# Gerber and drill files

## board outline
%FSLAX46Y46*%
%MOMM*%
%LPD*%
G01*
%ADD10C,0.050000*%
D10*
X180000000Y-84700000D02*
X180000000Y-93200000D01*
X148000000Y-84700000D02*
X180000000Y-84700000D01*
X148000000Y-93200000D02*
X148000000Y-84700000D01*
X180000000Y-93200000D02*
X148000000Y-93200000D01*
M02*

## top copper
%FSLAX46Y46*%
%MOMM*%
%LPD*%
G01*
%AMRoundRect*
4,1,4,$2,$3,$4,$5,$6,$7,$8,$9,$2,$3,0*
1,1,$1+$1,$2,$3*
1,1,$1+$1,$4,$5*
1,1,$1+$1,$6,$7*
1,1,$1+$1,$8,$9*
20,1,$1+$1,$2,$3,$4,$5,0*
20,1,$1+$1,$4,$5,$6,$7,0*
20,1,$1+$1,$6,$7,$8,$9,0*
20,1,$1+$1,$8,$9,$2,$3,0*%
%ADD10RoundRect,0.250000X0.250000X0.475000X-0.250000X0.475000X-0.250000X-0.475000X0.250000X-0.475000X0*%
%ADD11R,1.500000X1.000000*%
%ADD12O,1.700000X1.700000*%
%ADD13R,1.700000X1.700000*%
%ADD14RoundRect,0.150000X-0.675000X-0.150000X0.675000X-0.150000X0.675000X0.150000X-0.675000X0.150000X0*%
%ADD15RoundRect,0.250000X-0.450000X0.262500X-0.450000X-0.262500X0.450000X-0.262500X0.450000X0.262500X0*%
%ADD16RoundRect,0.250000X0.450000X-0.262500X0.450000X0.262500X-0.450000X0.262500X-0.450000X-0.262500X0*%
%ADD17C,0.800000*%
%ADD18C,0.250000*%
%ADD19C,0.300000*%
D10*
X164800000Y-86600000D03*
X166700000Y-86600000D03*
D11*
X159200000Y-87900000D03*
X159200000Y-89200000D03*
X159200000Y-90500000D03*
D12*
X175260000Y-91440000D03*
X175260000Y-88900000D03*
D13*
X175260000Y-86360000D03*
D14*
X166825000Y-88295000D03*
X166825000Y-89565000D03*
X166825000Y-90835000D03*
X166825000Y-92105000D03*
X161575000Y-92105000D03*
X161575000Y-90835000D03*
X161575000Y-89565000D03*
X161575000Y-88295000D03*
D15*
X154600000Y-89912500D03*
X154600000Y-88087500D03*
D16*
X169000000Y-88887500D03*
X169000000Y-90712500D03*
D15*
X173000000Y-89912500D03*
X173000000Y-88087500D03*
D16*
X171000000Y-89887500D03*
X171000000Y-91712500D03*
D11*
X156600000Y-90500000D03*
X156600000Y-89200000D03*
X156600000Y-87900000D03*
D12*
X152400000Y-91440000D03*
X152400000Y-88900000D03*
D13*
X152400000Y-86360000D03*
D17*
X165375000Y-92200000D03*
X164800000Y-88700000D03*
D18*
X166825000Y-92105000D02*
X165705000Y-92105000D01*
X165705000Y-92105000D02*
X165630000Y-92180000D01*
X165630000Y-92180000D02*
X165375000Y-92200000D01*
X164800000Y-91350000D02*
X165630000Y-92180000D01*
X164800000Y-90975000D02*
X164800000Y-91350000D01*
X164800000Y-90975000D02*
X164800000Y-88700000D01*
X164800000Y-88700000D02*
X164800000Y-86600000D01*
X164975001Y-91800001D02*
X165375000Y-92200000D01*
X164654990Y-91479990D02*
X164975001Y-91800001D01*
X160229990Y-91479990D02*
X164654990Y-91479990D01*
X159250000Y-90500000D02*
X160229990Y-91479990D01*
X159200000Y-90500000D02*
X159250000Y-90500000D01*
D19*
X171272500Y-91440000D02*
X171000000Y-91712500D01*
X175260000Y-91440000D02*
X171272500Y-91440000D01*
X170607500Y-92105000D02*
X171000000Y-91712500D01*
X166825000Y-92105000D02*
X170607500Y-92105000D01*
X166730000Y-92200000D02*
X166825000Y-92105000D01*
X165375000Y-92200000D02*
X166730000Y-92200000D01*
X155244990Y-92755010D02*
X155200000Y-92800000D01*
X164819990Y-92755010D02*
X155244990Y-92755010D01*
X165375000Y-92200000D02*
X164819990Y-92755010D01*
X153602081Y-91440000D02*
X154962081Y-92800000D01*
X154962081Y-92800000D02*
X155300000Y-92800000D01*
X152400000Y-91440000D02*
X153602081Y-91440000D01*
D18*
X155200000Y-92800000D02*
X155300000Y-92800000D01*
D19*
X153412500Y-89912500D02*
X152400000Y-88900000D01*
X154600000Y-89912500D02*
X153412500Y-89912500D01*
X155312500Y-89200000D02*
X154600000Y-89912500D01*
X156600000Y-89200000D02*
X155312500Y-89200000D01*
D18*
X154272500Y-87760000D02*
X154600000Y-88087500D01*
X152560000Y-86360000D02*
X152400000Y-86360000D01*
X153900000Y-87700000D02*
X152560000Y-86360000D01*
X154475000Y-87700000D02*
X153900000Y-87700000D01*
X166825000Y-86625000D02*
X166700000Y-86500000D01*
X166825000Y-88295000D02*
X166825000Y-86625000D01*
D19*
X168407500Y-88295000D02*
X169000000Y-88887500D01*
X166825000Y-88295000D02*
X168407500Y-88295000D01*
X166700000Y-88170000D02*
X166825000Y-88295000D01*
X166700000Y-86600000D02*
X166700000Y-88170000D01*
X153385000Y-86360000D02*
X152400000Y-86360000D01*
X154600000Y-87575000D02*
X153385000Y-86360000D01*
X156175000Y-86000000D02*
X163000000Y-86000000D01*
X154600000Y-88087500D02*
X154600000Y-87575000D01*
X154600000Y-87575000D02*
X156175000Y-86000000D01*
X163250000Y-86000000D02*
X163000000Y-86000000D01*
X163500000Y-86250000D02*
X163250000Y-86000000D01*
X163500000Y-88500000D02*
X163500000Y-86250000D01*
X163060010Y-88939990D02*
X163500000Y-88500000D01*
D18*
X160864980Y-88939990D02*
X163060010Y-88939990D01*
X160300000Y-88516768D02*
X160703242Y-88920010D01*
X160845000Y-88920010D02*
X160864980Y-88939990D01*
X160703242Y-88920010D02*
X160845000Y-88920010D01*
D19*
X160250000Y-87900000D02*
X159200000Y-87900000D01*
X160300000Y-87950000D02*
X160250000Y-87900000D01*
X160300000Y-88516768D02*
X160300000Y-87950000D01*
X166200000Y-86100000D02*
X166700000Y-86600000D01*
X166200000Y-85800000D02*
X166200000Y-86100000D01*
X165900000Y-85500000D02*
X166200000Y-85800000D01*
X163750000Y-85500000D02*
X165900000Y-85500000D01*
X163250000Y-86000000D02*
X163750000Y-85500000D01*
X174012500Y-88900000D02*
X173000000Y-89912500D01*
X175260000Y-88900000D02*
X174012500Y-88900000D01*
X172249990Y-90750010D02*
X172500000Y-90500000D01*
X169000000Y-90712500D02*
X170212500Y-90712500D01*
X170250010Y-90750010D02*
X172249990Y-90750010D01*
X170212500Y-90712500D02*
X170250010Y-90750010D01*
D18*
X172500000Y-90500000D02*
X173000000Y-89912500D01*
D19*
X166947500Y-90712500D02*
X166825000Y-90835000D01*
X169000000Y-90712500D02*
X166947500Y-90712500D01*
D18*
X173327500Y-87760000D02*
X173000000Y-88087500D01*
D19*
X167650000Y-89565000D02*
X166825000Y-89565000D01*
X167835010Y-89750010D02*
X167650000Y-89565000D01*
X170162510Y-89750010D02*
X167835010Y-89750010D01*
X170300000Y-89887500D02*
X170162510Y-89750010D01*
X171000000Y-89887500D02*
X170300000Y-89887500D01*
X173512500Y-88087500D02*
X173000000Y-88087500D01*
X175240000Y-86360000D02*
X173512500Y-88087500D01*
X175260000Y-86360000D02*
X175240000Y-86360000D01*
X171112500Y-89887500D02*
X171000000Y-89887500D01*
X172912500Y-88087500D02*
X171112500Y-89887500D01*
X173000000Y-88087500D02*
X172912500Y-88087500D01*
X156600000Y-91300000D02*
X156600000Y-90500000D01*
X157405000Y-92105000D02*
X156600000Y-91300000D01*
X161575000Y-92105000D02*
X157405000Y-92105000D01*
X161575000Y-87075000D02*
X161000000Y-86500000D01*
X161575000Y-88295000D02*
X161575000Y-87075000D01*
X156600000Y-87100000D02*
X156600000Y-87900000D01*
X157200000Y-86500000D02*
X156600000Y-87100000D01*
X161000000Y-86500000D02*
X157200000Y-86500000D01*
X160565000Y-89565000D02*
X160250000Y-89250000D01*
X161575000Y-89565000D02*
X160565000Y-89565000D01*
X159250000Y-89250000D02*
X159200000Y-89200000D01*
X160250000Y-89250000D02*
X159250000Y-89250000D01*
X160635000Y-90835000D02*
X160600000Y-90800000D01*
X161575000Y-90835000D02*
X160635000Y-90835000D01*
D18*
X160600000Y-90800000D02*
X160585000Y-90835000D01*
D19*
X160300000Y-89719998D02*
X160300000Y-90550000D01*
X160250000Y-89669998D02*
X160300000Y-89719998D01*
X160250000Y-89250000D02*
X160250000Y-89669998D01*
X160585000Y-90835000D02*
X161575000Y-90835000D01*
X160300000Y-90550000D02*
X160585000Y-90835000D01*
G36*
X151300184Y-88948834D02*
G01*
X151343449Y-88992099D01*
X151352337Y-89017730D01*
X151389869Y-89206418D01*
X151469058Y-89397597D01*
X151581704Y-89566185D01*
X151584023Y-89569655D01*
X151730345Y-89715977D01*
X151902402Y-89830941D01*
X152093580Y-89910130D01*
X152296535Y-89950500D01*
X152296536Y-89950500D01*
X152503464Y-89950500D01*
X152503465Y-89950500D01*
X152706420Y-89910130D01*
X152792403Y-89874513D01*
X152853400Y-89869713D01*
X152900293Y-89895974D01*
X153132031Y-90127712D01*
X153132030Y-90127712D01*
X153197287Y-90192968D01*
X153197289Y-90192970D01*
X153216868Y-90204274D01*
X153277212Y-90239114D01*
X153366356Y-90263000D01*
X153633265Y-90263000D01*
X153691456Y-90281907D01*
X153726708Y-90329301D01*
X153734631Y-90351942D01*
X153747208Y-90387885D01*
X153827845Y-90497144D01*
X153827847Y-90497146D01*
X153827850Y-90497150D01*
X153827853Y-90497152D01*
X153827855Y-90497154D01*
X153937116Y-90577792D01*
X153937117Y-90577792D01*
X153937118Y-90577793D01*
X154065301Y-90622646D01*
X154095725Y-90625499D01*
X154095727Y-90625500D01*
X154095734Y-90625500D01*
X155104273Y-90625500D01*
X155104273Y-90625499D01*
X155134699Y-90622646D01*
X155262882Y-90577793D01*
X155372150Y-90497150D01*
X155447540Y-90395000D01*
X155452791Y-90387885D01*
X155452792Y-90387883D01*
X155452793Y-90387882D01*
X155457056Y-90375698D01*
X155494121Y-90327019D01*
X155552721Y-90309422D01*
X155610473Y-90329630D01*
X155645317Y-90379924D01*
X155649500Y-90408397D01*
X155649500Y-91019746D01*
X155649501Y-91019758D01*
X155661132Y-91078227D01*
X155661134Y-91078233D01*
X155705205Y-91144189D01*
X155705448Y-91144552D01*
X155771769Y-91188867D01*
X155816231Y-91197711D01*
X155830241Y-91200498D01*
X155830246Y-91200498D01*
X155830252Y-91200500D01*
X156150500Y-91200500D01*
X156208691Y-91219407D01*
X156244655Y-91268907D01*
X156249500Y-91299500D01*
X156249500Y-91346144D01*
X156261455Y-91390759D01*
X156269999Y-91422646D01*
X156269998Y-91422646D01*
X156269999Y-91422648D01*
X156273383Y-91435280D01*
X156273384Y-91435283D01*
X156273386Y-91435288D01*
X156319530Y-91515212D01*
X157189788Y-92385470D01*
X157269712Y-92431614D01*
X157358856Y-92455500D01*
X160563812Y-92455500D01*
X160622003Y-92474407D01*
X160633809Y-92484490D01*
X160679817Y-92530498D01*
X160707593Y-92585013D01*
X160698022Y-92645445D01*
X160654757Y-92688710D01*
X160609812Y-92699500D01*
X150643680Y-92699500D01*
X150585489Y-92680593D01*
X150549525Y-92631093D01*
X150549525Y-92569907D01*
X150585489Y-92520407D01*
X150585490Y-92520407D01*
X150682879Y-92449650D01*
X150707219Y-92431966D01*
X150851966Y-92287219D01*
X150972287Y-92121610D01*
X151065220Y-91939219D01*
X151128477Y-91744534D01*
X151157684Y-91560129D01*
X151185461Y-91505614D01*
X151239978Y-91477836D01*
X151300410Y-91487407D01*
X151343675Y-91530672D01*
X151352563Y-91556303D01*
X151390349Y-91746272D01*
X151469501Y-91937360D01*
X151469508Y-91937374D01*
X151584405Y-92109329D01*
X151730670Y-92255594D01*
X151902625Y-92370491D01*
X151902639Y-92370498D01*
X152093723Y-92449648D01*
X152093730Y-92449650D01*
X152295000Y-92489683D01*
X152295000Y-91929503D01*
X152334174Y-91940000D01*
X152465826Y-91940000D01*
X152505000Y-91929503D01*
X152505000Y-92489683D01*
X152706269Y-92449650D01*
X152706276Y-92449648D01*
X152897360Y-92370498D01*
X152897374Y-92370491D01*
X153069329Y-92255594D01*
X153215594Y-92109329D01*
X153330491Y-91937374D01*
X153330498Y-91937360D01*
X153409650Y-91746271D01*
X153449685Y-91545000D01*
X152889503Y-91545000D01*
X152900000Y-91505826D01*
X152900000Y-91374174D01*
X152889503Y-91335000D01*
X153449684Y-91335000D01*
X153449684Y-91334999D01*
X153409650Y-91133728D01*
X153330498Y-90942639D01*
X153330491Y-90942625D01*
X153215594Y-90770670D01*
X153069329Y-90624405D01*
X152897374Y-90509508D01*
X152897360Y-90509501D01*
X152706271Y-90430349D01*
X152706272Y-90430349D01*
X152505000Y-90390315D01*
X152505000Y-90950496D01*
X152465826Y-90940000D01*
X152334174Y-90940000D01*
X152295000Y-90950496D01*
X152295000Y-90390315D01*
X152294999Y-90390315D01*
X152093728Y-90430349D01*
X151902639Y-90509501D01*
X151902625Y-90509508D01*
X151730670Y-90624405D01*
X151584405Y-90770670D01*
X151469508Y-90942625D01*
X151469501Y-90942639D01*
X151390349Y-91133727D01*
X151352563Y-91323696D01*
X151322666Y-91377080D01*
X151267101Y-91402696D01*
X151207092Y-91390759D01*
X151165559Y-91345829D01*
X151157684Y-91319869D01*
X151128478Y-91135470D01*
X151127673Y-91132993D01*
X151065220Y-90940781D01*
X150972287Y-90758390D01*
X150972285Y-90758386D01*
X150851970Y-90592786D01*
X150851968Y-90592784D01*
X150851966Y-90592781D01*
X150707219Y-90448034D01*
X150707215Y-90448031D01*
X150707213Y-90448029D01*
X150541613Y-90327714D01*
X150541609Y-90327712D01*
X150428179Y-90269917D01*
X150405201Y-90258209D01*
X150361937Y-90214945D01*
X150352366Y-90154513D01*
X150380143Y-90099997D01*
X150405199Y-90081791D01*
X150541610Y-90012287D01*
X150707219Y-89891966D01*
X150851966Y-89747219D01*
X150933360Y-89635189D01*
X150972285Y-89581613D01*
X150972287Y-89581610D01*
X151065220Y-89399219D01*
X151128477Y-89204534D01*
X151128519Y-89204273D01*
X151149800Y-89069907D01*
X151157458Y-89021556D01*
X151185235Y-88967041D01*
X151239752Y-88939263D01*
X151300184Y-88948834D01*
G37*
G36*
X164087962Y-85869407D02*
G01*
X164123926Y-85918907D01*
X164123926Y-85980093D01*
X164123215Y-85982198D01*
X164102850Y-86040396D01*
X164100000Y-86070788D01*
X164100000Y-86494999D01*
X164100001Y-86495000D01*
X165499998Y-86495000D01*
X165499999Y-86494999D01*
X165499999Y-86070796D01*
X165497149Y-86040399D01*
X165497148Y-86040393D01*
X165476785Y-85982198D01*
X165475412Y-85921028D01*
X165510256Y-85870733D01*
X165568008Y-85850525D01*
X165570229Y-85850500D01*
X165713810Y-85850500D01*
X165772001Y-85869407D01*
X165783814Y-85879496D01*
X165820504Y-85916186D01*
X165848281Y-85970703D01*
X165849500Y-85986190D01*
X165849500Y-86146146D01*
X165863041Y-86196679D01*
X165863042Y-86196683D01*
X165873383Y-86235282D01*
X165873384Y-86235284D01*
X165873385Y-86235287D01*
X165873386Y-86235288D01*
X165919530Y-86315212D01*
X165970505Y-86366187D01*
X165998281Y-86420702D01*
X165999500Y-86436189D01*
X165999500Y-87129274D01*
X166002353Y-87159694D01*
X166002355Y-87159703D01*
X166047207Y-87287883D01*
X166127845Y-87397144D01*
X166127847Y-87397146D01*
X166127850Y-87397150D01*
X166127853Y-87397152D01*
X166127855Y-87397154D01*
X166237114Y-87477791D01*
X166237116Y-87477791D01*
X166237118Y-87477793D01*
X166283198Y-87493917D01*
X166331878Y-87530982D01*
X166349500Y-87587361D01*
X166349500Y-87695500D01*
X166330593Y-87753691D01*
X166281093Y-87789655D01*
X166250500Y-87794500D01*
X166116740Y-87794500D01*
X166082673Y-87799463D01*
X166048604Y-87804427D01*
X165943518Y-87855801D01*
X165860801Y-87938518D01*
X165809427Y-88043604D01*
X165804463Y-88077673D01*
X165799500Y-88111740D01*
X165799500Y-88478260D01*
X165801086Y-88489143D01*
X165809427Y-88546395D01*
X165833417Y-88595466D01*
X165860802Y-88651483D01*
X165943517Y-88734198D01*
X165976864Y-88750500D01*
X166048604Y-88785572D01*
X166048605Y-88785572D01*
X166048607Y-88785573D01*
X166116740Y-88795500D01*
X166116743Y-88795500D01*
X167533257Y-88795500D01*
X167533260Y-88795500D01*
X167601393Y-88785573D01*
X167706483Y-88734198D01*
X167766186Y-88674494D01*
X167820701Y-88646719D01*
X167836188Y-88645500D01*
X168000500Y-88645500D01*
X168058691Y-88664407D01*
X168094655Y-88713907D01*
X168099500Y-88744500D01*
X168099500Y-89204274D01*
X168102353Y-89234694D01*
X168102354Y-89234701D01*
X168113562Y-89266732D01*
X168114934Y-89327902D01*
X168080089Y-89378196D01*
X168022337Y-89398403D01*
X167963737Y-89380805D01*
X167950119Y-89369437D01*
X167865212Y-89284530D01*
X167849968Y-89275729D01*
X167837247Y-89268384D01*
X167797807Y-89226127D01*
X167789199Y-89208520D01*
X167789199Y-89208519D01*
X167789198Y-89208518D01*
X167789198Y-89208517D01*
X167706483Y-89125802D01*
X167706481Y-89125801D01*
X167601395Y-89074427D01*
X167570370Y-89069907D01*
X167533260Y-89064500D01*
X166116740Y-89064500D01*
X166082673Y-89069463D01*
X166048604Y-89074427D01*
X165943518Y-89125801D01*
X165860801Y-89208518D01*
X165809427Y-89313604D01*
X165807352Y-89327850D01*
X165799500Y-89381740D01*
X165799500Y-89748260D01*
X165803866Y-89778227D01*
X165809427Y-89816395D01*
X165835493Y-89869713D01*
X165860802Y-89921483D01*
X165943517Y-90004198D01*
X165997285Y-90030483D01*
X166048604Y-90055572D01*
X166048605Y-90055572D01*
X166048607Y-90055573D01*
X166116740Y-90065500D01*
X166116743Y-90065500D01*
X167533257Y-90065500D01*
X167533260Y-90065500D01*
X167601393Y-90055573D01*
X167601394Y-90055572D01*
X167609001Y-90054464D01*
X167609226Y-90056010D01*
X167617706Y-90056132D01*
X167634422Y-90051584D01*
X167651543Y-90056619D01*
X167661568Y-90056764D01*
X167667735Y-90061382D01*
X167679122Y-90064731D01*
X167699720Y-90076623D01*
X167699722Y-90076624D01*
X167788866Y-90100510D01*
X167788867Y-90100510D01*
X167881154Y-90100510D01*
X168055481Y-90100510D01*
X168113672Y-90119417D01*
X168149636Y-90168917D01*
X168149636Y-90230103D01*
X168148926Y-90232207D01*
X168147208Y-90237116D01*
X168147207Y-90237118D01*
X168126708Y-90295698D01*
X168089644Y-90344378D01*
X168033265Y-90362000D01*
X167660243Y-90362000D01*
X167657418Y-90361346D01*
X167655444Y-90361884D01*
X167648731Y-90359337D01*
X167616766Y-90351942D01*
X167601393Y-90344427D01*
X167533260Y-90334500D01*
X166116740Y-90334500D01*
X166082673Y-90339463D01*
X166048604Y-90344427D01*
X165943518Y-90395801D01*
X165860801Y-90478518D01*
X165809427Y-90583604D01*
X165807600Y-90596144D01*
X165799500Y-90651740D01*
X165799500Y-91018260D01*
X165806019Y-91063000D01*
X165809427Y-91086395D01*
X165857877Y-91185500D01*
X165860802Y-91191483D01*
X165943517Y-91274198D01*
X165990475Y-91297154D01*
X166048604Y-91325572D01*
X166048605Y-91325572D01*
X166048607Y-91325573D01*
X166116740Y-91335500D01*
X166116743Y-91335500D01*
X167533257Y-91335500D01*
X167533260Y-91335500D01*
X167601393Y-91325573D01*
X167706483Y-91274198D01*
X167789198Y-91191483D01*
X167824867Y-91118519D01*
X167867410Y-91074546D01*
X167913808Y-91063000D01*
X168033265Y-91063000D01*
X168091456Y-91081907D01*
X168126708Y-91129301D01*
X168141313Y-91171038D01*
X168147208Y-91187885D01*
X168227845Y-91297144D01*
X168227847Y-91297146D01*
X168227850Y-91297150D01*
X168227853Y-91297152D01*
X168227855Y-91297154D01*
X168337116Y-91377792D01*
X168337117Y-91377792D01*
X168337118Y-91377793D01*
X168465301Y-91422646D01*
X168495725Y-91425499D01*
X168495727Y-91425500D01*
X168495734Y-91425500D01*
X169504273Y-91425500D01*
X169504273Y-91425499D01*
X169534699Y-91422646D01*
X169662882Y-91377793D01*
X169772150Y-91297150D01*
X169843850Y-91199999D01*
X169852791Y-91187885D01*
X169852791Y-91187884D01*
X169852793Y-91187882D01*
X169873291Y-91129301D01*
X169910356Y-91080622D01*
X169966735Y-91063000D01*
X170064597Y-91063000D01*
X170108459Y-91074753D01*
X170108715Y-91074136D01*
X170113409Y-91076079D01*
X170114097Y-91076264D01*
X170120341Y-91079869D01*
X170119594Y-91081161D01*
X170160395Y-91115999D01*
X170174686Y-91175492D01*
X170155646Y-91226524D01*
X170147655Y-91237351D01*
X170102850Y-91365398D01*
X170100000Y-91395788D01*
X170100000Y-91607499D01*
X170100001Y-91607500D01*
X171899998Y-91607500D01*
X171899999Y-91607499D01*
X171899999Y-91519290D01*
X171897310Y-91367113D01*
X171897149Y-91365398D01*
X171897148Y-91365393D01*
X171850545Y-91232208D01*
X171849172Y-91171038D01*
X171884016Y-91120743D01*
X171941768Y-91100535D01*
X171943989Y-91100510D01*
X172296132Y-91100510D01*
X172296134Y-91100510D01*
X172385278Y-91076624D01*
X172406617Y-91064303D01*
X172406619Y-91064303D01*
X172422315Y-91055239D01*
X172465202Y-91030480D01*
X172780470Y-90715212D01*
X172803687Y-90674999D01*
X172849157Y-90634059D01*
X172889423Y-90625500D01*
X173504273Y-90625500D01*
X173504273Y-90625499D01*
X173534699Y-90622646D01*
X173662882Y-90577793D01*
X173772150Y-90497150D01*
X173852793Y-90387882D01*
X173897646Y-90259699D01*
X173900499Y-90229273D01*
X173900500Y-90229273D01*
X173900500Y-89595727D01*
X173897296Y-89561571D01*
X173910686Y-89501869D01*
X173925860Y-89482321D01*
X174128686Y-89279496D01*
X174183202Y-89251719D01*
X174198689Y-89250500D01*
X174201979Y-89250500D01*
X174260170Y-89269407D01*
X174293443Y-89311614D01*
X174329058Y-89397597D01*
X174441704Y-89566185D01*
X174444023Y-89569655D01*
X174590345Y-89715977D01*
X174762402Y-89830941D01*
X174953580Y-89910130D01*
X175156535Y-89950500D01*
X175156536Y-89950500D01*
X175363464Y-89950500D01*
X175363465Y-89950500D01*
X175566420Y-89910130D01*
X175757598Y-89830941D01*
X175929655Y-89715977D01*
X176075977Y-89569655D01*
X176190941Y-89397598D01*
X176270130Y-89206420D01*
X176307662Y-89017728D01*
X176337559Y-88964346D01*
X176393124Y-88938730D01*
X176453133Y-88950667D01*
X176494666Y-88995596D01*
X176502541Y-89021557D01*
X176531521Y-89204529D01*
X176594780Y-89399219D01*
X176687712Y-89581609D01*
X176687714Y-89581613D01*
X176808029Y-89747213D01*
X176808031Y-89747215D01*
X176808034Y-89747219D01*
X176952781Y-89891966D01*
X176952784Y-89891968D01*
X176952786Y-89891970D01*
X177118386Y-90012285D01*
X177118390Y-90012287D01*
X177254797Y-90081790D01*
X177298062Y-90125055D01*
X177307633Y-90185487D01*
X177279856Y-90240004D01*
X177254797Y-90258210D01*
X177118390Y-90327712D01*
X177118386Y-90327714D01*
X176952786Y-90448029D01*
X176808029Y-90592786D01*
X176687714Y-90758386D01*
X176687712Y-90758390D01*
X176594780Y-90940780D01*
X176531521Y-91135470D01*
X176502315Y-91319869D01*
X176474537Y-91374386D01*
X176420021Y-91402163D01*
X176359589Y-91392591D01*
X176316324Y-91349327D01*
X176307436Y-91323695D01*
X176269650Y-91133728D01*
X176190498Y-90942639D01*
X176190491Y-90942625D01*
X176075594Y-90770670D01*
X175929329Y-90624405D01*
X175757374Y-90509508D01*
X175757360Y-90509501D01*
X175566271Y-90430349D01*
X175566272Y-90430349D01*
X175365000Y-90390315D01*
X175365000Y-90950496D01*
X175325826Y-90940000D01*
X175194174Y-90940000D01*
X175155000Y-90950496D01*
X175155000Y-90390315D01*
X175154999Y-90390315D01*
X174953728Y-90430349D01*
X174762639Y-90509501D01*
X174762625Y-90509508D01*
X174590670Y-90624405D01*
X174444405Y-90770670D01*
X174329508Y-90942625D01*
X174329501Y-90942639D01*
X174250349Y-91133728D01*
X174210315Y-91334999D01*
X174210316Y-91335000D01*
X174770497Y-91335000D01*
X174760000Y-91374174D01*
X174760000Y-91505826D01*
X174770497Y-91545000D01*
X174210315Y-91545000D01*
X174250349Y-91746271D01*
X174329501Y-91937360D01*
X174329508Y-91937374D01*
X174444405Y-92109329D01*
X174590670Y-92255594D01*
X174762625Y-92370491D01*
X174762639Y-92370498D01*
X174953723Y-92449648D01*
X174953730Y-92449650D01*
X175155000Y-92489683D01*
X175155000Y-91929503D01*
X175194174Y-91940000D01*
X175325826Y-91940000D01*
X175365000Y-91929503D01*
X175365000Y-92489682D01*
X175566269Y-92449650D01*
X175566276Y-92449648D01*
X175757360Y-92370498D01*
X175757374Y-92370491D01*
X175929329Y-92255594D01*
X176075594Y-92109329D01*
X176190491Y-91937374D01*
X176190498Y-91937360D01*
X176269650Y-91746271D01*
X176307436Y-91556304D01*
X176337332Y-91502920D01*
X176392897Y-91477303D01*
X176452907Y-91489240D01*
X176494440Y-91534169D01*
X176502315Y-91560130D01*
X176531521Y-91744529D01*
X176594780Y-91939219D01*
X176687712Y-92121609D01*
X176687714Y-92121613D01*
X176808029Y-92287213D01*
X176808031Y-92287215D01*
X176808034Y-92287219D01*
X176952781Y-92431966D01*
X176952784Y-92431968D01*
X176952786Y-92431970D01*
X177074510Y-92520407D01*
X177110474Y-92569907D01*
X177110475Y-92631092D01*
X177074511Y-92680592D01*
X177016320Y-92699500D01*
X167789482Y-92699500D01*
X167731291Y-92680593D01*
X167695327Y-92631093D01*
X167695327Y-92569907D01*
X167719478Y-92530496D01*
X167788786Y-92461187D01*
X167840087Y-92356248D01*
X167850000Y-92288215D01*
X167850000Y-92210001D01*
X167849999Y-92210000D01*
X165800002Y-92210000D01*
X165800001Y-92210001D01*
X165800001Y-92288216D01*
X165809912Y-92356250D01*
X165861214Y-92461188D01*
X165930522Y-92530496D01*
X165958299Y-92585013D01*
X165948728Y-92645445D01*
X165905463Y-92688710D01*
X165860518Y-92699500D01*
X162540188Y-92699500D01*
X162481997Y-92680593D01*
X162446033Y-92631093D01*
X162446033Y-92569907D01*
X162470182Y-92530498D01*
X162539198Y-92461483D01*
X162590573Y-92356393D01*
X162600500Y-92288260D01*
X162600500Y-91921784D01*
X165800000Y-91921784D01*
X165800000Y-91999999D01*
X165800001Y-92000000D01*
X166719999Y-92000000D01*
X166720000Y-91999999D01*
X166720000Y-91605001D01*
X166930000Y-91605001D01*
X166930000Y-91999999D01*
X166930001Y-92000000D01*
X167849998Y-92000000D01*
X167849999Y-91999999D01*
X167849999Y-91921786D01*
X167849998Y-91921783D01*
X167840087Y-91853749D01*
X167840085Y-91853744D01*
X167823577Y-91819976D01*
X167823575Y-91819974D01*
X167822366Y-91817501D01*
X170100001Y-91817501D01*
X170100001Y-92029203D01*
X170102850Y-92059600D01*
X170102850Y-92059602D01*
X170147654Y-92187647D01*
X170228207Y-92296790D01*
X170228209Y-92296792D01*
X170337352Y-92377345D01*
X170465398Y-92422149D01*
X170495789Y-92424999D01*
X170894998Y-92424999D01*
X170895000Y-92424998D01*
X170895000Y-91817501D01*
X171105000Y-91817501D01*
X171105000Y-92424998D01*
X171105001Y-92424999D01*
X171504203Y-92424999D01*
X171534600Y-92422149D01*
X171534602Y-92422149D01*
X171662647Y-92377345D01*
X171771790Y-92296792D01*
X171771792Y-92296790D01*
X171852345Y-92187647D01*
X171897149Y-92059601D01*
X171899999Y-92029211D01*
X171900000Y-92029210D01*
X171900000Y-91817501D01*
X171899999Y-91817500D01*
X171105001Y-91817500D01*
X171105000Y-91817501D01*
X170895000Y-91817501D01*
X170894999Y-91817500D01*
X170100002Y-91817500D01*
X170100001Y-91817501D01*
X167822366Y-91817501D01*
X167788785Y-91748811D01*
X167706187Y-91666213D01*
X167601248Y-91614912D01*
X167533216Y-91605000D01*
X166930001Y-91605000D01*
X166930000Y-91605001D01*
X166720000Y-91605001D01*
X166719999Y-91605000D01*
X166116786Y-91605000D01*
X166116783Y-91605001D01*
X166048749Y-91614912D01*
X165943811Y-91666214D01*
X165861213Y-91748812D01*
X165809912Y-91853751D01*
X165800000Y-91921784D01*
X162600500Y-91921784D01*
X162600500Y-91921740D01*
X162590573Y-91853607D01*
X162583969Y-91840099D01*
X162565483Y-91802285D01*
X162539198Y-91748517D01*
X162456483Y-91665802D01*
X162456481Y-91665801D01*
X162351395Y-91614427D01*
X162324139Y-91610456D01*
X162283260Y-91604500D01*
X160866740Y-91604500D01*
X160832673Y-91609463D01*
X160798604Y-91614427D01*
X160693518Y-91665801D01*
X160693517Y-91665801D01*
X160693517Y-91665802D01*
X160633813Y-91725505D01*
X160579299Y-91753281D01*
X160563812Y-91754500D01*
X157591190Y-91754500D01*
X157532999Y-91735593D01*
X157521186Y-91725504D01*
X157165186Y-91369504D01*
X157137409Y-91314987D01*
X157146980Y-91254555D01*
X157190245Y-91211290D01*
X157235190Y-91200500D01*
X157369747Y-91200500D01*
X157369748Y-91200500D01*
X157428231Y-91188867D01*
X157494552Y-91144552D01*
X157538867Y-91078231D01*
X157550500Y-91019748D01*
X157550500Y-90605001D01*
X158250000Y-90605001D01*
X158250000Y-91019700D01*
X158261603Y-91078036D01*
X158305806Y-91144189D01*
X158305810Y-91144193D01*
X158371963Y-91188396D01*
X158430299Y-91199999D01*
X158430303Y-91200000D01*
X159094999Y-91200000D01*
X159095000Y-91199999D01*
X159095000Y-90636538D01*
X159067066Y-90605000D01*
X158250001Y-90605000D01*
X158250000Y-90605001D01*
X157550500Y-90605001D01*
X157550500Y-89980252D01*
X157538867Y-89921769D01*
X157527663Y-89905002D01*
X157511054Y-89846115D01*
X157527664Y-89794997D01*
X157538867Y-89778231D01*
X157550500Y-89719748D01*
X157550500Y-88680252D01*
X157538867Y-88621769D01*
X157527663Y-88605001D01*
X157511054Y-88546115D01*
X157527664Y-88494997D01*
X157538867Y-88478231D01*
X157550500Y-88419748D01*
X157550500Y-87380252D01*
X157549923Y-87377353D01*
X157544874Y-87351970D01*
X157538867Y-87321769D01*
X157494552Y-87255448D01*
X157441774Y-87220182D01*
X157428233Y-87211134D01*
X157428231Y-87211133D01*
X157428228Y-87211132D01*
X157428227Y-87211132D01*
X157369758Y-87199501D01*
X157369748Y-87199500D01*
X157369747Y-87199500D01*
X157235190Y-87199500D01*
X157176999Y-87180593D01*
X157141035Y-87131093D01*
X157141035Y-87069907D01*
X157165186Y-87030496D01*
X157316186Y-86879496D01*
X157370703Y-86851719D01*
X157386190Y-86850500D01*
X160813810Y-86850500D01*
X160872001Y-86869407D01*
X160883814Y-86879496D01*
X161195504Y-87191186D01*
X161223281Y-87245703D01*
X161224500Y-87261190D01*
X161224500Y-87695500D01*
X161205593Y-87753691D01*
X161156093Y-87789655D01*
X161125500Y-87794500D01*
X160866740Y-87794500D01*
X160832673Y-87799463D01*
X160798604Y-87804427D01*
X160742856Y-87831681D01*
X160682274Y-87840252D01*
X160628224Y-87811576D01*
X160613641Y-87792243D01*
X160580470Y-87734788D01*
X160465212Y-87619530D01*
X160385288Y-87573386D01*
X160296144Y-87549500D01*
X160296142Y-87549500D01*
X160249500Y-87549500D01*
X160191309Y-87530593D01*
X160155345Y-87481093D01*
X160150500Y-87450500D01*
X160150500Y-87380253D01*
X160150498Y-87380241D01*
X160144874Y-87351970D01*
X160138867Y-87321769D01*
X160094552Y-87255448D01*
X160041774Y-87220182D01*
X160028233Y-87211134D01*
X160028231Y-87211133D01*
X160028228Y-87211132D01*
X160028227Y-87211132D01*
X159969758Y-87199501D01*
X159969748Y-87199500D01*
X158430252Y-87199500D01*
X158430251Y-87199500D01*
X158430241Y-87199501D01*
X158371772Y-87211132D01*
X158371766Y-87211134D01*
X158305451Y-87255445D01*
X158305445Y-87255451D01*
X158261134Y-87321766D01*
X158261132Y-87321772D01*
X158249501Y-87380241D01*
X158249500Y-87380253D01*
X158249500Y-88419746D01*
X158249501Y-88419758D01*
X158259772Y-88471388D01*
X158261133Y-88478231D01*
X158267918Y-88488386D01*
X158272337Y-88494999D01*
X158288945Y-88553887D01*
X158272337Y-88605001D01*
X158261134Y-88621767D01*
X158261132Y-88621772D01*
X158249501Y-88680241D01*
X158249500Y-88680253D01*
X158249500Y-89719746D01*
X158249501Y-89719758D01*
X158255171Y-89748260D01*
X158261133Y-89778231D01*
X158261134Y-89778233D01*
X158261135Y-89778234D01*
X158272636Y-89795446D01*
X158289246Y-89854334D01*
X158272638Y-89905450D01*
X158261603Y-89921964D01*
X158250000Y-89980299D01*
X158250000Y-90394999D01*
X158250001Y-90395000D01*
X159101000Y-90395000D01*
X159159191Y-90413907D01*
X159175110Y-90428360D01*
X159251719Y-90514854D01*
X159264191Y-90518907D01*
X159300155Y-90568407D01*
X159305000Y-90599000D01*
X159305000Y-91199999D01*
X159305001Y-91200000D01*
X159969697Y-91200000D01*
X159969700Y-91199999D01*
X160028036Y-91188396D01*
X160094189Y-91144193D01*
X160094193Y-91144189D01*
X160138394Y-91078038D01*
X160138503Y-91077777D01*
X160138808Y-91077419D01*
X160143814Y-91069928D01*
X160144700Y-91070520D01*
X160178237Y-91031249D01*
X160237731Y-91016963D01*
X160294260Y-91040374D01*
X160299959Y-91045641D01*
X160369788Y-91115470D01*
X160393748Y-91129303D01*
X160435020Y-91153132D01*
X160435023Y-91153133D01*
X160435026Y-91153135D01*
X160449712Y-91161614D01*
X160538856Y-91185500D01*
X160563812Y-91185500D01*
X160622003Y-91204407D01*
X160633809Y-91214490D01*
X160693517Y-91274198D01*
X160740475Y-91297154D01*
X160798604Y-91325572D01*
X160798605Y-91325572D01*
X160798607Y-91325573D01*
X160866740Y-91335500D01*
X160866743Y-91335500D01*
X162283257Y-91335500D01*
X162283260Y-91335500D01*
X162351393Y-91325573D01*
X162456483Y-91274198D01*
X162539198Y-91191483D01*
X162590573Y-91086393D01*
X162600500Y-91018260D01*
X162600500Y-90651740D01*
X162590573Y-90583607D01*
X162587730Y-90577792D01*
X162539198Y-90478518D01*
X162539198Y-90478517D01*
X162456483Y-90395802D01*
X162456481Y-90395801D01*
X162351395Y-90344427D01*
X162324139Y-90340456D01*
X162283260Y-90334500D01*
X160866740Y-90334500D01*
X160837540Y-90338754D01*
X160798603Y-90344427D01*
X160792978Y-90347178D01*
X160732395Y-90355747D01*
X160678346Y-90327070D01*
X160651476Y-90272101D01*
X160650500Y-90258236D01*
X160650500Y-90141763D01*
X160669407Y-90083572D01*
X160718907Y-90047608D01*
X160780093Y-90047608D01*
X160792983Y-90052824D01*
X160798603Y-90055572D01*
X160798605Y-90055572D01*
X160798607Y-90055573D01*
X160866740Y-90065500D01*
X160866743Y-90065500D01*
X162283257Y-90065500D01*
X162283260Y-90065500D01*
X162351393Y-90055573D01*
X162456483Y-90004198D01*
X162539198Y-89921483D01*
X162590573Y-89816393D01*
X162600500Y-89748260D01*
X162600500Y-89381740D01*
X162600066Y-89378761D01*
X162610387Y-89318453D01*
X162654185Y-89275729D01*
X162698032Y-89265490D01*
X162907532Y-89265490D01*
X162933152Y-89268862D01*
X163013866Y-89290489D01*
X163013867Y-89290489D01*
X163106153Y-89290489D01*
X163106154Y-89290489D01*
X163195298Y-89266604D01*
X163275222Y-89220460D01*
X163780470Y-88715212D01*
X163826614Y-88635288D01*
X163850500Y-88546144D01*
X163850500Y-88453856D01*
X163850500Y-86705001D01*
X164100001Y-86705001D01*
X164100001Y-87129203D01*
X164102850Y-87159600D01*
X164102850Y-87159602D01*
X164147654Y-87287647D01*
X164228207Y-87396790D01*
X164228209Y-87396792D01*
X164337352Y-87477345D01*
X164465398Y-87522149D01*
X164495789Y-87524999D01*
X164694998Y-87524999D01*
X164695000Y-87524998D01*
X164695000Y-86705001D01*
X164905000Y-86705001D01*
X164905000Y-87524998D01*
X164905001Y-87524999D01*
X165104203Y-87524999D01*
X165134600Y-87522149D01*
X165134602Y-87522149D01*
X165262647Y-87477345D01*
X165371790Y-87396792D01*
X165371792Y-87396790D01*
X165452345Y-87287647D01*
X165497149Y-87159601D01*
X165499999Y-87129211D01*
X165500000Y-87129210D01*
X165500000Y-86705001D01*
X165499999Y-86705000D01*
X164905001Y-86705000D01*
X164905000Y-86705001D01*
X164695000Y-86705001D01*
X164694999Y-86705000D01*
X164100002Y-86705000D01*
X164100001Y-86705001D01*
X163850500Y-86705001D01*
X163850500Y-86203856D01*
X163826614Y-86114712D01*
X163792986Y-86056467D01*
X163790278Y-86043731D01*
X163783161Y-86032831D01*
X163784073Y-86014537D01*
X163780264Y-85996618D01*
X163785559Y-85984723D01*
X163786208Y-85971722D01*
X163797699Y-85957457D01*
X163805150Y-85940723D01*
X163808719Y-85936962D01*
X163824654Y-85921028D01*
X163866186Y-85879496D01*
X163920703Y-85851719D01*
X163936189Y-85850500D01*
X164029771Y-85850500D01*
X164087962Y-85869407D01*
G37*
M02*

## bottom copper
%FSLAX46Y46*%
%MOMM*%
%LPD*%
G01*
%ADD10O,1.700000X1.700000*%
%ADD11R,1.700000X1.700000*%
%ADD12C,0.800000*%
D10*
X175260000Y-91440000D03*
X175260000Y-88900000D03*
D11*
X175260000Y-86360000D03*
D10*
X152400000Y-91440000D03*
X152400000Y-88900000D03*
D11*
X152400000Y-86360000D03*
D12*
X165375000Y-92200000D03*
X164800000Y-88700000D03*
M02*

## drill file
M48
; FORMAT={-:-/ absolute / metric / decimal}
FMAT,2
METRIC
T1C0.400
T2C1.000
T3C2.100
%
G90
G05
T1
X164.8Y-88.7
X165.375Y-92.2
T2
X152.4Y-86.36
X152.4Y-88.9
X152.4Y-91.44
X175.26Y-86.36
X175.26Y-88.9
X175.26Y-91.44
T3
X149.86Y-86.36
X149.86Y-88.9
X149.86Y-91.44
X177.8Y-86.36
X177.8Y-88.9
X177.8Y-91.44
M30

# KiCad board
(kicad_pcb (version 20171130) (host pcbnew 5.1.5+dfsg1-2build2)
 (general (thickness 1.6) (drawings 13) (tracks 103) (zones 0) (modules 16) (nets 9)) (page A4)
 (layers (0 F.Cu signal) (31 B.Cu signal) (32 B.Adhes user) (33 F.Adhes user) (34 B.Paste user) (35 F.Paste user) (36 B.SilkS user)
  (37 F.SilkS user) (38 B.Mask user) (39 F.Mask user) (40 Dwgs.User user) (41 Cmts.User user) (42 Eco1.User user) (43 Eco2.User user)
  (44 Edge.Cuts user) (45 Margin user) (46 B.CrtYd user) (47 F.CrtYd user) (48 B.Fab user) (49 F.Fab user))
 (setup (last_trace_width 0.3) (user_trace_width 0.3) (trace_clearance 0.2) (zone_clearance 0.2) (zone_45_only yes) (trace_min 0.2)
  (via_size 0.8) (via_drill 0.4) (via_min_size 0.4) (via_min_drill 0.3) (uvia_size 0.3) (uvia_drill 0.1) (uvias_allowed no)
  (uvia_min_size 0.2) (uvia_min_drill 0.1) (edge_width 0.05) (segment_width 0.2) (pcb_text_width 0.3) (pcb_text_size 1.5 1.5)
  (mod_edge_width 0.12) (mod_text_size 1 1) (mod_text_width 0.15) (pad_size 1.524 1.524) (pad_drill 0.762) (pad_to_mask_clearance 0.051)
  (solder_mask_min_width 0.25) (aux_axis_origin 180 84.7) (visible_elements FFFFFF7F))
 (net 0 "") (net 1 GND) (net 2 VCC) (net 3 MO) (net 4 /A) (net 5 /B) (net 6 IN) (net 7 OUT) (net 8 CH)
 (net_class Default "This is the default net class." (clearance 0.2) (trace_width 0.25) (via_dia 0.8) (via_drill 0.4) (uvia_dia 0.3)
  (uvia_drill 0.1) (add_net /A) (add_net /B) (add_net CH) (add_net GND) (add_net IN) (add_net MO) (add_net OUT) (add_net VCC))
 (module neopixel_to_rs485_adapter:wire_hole (layer F.Cu) (at 177.8 91.44)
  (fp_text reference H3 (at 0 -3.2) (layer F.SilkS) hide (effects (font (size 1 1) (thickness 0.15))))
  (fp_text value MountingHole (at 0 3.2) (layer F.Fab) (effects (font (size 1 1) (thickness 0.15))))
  (pad "" np_thru_hole circle (at 0 0) (size 2.1 2.1) (drill 2.1) (layers *.Cu *.Mask)))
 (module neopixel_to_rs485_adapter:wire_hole (layer F.Cu) (at 177.8 88.9)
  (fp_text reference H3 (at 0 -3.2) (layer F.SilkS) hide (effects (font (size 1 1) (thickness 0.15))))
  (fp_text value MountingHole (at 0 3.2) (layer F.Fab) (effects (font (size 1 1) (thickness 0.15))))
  (pad "" np_thru_hole circle (at 0 0) (size 2.1 2.1) (drill 2.1) (layers *.Cu *.Mask)))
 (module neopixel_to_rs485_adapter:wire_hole (layer F.Cu) (at 177.8 86.36)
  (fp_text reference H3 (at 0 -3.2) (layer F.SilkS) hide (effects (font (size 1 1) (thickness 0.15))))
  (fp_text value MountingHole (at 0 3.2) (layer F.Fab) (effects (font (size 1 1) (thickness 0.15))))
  (pad "" np_thru_hole circle (at 0 0) (size 2.1 2.1) (drill 2.1) (layers *.Cu *.Mask)))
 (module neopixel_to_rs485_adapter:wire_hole (layer F.Cu) (at 149.86 91.44)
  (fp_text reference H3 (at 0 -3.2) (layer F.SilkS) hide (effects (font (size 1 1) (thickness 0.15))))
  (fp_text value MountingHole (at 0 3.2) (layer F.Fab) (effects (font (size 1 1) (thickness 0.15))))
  (pad "" np_thru_hole circle (at 0 0) (size 2.1 2.1) (drill 2.1) (layers *.Cu *.Mask)))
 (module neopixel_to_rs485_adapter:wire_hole (layer F.Cu) (at 149.86 88.9)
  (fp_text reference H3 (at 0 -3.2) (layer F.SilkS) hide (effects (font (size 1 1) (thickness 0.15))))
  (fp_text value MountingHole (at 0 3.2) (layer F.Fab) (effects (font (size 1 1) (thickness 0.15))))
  (pad "" np_thru_hole circle (at 0 0) (size 2.1 2.1) (drill 2.1) (layers *.Cu *.Mask)))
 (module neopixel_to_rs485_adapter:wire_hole (layer F.Cu) (at 149.86 86.36)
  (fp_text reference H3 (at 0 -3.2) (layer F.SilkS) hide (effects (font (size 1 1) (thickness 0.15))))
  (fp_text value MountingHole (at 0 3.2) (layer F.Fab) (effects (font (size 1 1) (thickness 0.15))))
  (pad "" np_thru_hole circle (at 0 0) (size 2.1 2.1) (drill 2.1) (layers *.Cu *.Mask)))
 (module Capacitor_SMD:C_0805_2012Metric (layer F.Cu) (at 165.75 86.6 180)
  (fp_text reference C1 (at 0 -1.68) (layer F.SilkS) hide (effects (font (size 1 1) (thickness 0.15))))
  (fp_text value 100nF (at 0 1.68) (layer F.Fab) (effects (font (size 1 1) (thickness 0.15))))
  (pad 2 smd roundrect (at 0.95 0 180) (size 1 1.45) (layers F.Cu F.Paste F.Mask) (roundrect_rratio 0.25) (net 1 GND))
  (pad 1 smd roundrect (at -0.95 0 180) (size 1 1.45) (layers F.Cu F.Paste F.Mask) (roundrect_rratio 0.25) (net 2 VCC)))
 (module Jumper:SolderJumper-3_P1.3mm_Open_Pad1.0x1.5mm (layer F.Cu) (at 159.2 89.2 270)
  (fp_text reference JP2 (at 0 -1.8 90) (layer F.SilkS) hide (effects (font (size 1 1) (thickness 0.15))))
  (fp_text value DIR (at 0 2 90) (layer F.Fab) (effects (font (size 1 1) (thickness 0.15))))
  (pad 1 smd rect (at -1.3 0 270) (size 1 1.5) (layers F.Cu F.Mask) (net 2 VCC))
  (pad 2 smd rect (at 0 0 270) (size 1 1.5) (layers F.Cu F.Mask) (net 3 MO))
  (pad 3 smd rect (at 1.3 0 270) (size 1 1.5) (layers F.Cu F.Mask) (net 1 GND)))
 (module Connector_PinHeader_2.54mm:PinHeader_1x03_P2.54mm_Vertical (layer F.Cu) (at 175.26 86.36)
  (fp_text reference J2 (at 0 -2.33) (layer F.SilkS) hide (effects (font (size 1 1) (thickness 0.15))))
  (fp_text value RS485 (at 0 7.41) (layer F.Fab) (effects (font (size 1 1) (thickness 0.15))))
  (pad 3 thru_hole oval (at 0 5.08) (size 1.7 1.7) (drill 1) (layers *.Cu *.Mask) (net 1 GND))
  (pad 2 thru_hole oval (at 0 2.54) (size 1.7 1.7) (drill 1) (layers *.Cu *.Mask) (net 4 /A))
  (pad 1 thru_hole rect (at 0 0) (size 1.7 1.7) (drill 1) (layers *.Cu *.Mask) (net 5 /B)))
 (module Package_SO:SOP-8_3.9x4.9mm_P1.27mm (layer F.Cu) (at 164.2 90.2)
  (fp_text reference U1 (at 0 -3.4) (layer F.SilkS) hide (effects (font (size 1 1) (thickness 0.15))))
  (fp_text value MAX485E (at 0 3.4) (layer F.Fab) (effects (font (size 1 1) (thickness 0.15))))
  (pad 8 smd roundrect (at 2.625 -1.905) (size 1.65 0.6) (layers F.Cu F.Paste F.Mask) (roundrect_rratio 0.25) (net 2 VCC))
  (pad 7 smd roundrect (at 2.625 -0.635) (size 1.65 0.6) (layers F.Cu F.Paste F.Mask) (roundrect_rratio 0.25) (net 5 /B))
  (pad 6 smd roundrect (at 2.625 0.635) (size 1.65 0.6) (layers F.Cu F.Paste F.Mask) (roundrect_rratio 0.25) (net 4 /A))
  (pad 5 smd roundrect (at 2.625 1.905) (size 1.65 0.6) (layers F.Cu F.Paste F.Mask) (roundrect_rratio 0.25) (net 1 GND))
  (pad 4 smd roundrect (at -2.625 1.905) (size 1.65 0.6) (layers F.Cu F.Paste F.Mask) (roundrect_rratio 0.25) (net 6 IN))
  (pad 3 smd roundrect (at -2.625 0.635) (size 1.65 0.6) (layers F.Cu F.Paste F.Mask) (roundrect_rratio 0.25) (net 3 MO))
  (pad 2 smd roundrect (at -2.625 -0.635) (size 1.65 0.6) (layers F.Cu F.Paste F.Mask) (roundrect_rratio 0.25) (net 3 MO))
  (pad 1 smd roundrect (at -2.625 -1.905) (size 1.65 0.6) (layers F.Cu F.Paste F.Mask) (roundrect_rratio 0.25) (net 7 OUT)))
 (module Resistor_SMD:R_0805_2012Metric (layer F.Cu) (at 154.6 89 270)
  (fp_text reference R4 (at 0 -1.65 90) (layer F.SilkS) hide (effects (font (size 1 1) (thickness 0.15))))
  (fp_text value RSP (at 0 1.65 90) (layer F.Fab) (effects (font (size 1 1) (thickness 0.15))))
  (pad 2 smd roundrect (at 0.9125 0 270) (size 1.025 1.4) (layers F.Cu F.Paste F.Mask) (roundrect_rratio 0.243902) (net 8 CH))
  (pad 1 smd roundrect (at -0.9125 0 270) (size 1.025 1.4) (layers F.Cu F.Paste F.Mask) (roundrect_rratio 0.243902) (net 2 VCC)))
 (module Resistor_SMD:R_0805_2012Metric (layer F.Cu) (at 169 89.8 90)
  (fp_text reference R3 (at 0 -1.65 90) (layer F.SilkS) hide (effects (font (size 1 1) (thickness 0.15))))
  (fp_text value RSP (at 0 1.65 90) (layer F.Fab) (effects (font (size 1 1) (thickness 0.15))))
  (pad 2 smd roundrect (at 0.9125 0 90) (size 1.025 1.4) (layers F.Cu F.Paste F.Mask) (roundrect_rratio 0.243902) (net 2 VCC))
  (pad 1 smd roundrect (at -0.9125 0 90) (size 1.025 1.4) (layers F.Cu F.Paste F.Mask) (roundrect_rratio 0.243902) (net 4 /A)))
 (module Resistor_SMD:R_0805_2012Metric (layer F.Cu) (at 173 89 270)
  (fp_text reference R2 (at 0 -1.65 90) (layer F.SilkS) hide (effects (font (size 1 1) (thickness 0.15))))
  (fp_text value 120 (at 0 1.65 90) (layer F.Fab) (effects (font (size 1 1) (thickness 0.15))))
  (pad 2 smd roundrect (at 0.9125 0 270) (size 1.025 1.4) (layers F.Cu F.Paste F.Mask) (roundrect_rratio 0.243902) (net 4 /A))
  (pad 1 smd roundrect (at -0.9125 0 270) (size 1.025 1.4) (layers F.Cu F.Paste F.Mask) (roundrect_rratio 0.243902) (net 5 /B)))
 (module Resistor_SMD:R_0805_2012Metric (layer F.Cu) (at 171 90.8 90)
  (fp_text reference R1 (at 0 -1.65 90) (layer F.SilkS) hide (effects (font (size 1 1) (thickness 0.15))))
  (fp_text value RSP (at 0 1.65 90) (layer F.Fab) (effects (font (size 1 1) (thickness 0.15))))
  (pad 2 smd roundrect (at 0.9125 0 90) (size 1.025 1.4) (layers F.Cu F.Paste F.Mask) (roundrect_rratio 0.243902) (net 5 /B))
  (pad 1 smd roundrect (at -0.9125 0 90) (size 1.025 1.4) (layers F.Cu F.Paste F.Mask) (roundrect_rratio 0.243902) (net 1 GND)))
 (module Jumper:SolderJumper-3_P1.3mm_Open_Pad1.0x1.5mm (layer F.Cu) (at 156.6 89.2 90)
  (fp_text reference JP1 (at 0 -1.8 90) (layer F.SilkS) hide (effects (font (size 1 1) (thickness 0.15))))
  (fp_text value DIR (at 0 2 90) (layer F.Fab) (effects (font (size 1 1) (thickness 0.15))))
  (pad 1 smd rect (at -1.3 0 90) (size 1 1.5) (layers F.Cu F.Mask) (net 6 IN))
  (pad 2 smd rect (at 0 0 90) (size 1 1.5) (layers F.Cu F.Mask) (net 8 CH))
  (pad 3 smd rect (at 1.3 0 90) (size 1 1.5) (layers F.Cu F.Mask) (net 7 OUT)))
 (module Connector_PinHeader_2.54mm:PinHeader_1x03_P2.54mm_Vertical (layer F.Cu) (at 152.4 86.36)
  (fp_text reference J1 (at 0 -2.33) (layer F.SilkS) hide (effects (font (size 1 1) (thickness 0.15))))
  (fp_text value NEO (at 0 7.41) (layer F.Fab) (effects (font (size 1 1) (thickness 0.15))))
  (pad 3 thru_hole oval (at 0 5.08) (size 1.7 1.7) (drill 1) (layers *.Cu *.Mask) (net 1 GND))
  (pad 2 thru_hole oval (at 0 2.54) (size 1.7 1.7) (drill 1) (layers *.Cu *.Mask) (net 8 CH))
  (pad 1 thru_hole rect (at 0 0) (size 1.7 1.7) (drill 1) (layers *.Cu *.Mask) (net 2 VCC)))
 (gr_line (start 180 84.7) (end 180 93.2) (layer Edge.Cuts) (width 0.05))
 (gr_line (start 148 84.7) (end 180 84.7) (layer Edge.Cuts) (width 0.05))
 (gr_line (start 148 93.2) (end 148 84.7) (layer Edge.Cuts) (width 0.05))
 (gr_line (start 180 93.2) (end 148 93.2) (layer Edge.Cuts) (width 0.05))
 (segment (start 166.825 92.105) (end 165.705 92.105) (width 0.25) (layer F.Cu) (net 1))
 (segment (start 165.705 92.105) (end 165.63 92.18) (width 0.25) (layer F.Cu) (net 1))
 (segment (start 165.63 92.18) (end 165.375 92.2) (width 0.25) (layer F.Cu) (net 1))
 (segment (start 164.8 91.35) (end 165.63 92.18) (width 0.25) (layer F.Cu) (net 1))
 (segment (start 164.8 90.975) (end 164.8 91.35) (width 0.25) (layer F.Cu) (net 1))
 (segment (start 164.8 90.975) (end 164.8 88.7) (width 0.25) (layer F.Cu) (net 1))
 (via (at 165.375 92.2) (size 0.8) (drill 0.4) (layers F.Cu B.Cu) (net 1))
 (segment (start 164.8 88.7) (end 164.8 86.6) (width 0.25) (layer F.Cu) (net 1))
 (via (at 164.8 88.7) (size 0.8) (drill 0.4) (layers F.Cu B.Cu) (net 1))
 (segment (start 164.975001 91.800001) (end 165.375 92.2) (width 0.25) (layer F.Cu) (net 1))
 (segment (start 164.65499 91.47999) (end 164.975001 91.800001) (width 0.25) (layer F.Cu) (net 1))
 (segment (start 160.22999 91.47999) (end 164.65499 91.47999) (width 0.25) (layer F.Cu) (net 1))
 (segment (start 159.25 90.5) (end 160.22999 91.47999) (width 0.25) (layer F.Cu) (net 1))
 (segment (start 159.2 90.5) (end 159.25 90.5) (width 0.25) (layer F.Cu) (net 1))
 (segment (start 171.2725 91.44) (end 171 91.7125) (width 0.3) (layer F.Cu) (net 1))
 (segment (start 175.26 91.44) (end 171.2725 91.44) (width 0.3) (layer F.Cu) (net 1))
 (segment (start 170.6075 92.105) (end 171 91.7125) (width 0.3) (layer F.Cu) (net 1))
 (segment (start 166.825 92.105) (end 170.6075 92.105) (width 0.3) (layer F.Cu) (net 1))
 (segment (start 166.73 92.2) (end 166.825 92.105) (width 0.3) (layer F.Cu) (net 1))
 (segment (start 165.375 92.2) (end 166.73 92.2) (width 0.3) (layer F.Cu) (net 1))
 (segment (start 155.24499 92.75501) (end 155.2 92.8) (width 0.3) (layer F.Cu) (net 1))
 (segment (start 164.81999 92.75501) (end 155.24499 92.75501) (width 0.3) (layer F.Cu) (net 1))
 (segment (start 165.375 92.2) (end 164.81999 92.75501) (width 0.3) (layer F.Cu) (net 1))
 (segment (start 153.602081 91.44) (end 154.962081 92.8) (width 0.3) (layer F.Cu) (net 1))
 (segment (start 154.962081 92.8) (end 155.3 92.8) (width 0.3) (layer F.Cu) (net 1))
 (segment (start 152.4 91.44) (end 153.602081 91.44) (width 0.3) (layer F.Cu) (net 1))
 (segment (start 155.2 92.8) (end 155.3 92.8) (width 0.25) (layer F.Cu) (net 1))
 (segment (start 153.4125 89.9125) (end 152.4 88.9) (width 0.3) (layer F.Cu) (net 8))
 (segment (start 154.6 89.9125) (end 153.4125 89.9125) (width 0.3) (layer F.Cu) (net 8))
 (segment (start 155.3125 89.2) (end 154.6 89.9125) (width 0.3) (layer F.Cu) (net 8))
 (segment (start 156.6 89.2) (end 155.3125 89.2) (width 0.3) (layer F.Cu) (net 8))
 (segment (start 154.2725 87.76) (end 154.6 88.0875) (width 0.25) (layer F.Cu) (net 2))
 (segment (start 152.56 86.36) (end 152.4 86.36) (width 0.25) (layer F.Cu) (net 2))
 (segment (start 153.9 87.7) (end 152.56 86.36) (width 0.25) (layer F.Cu) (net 2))
 (segment (start 154.475 87.7) (end 153.9 87.7) (width 0.25) (layer F.Cu) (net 2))
 (segment (start 166.825 86.625) (end 166.7 86.5) (width 0.25) (layer F.Cu) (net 2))
 (segment (start 166.825 88.295) (end 166.825 86.625) (width 0.25) (layer F.Cu) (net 2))
 (segment (start 168.4075 88.295) (end 169 88.8875) (width 0.3) (layer F.Cu) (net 2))
 (segment (start 166.825 88.295) (end 168.4075 88.295) (width 0.3) (layer F.Cu) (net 2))
 (segment (start 166.7 88.17) (end 166.825 88.295) (width 0.3) (layer F.Cu) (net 2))
 (segment (start 166.7 86.6) (end 166.7 88.17) (width 0.3) (layer F.Cu) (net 2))
 (segment (start 153.385 86.36) (end 152.4 86.36) (width 0.3) (layer F.Cu) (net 2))
 (segment (start 154.6 87.575) (end 153.385 86.36) (width 0.3) (layer F.Cu) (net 2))
 (segment (start 156.175 86) (end 163 86) (width 0.3) (layer F.Cu) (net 2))
 (segment (start 154.6 88.0875) (end 154.6 87.575) (width 0.3) (layer F.Cu) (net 2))
 (segment (start 154.6 87.575) (end 156.175 86) (width 0.3) (layer F.Cu) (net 2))
 (segment (start 163.25 86) (end 163 86) (width 0.3) (layer F.Cu) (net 2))
 (segment (start 163.5 86.25) (end 163.25 86) (width 0.3) (layer F.Cu) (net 2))
 (segment (start 163.5 88.5) (end 163.5 86.25) (width 0.3) (layer F.Cu) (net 2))
 (segment (start 163.06001 88.93999) (end 163.5 88.5) (width 0.3) (layer F.Cu) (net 2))
 (segment (start 160.86498 88.93999) (end 163.06001 88.93999) (width 0.25) (layer F.Cu) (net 2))
 (segment (start 160.3 88.516768) (end 160.703242 88.92001) (width 0.25) (layer F.Cu) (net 2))
 (segment (start 160.845 88.92001) (end 160.86498 88.93999) (width 0.25) (layer F.Cu) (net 2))
 (segment (start 160.703242 88.92001) (end 160.845 88.92001) (width 0.25) (layer F.Cu) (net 2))
 (segment (start 160.25 87.9) (end 159.2 87.9) (width 0.3) (layer F.Cu) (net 2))
 (segment (start 160.3 87.95) (end 160.25 87.9) (width 0.3) (layer F.Cu) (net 2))
 (segment (start 160.3 88.516768) (end 160.3 87.95) (width 0.3) (layer F.Cu) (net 2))
 (segment (start 166.2 86.1) (end 166.7 86.6) (width 0.3) (layer F.Cu) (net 2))
 (segment (start 166.2 85.8) (end 166.2 86.1) (width 0.3) (layer F.Cu) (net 2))
 (segment (start 165.9 85.5) (end 166.2 85.8) (width 0.3) (layer F.Cu) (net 2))
 (segment (start 163.75 85.5) (end 165.9 85.5) (width 0.3) (layer F.Cu) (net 2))
 (segment (start 163.25 86) (end 163.75 85.5) (width 0.3) (layer F.Cu) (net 2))
 (segment (start 174.0125 88.9) (end 173 89.9125) (width 0.3) (layer F.Cu) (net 4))
 (segment (start 175.26 88.9) (end 174.0125 88.9) (width 0.3) (layer F.Cu) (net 4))
 (segment (start 172.24999 90.75001) (end 172.5 90.5) (width 0.3) (layer F.Cu) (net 4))
 (segment (start 169 90.7125) (end 170.2125 90.7125) (width 0.3) (layer F.Cu) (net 4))
 (segment (start 170.25001 90.75001) (end 172.24999 90.75001) (width 0.3) (layer F.Cu) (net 4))
 (segment (start 170.2125 90.7125) (end 170.25001 90.75001) (width 0.3) (layer F.Cu) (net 4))
 (segment (start 172.5 90.5) (end 173 89.9125) (width 0.25) (layer F.Cu) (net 4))
 (segment (start 166.9475 90.7125) (end 166.825 90.835) (width 0.3) (layer F.Cu) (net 4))
 (segment (start 169 90.7125) (end 166.9475 90.7125) (width 0.3) (layer F.Cu) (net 4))
 (segment (start 173.3275 87.76) (end 173 88.0875) (width 0.25) (layer F.Cu) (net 5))
 (segment (start 167.65 89.565) (end 166.825 89.565) (width 0.3) (layer F.Cu) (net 5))
 (segment (start 167.83501 89.75001) (end 167.65 89.565) (width 0.3) (layer F.Cu) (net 5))
 (segment (start 170.16251 89.75001) (end 167.83501 89.75001) (width 0.3) (layer F.Cu) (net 5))
 (segment (start 170.3 89.8875) (end 170.16251 89.75001) (width 0.3) (layer F.Cu) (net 5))
 (segment (start 171 89.8875) (end 170.3 89.8875) (width 0.3) (layer F.Cu) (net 5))
 (segment (start 173.5125 88.0875) (end 173 88.0875) (width 0.3) (layer F.Cu) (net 5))
 (segment (start 175.24 86.36) (end 173.5125 88.0875) (width 0.3) (layer F.Cu) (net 5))
 (segment (start 175.26 86.36) (end 175.24 86.36) (width 0.3) (layer F.Cu) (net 5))
 (segment (start 171.1125 89.8875) (end 171 89.8875) (width 0.3) (layer F.Cu) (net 5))
 (segment (start 172.9125 88.0875) (end 171.1125 89.8875) (width 0.3) (layer F.Cu) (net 5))
 (segment (start 173 88.0875) (end 172.9125 88.0875) (width 0.3) (layer F.Cu) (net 5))
 (segment (start 156.6 91.3) (end 156.6 90.5) (width 0.3) (layer F.Cu) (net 6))
 (segment (start 157.405 92.105) (end 156.6 91.3) (width 0.3) (layer F.Cu) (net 6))
 (segment (start 161.575 92.105) (end 157.405 92.105) (width 0.3) (layer F.Cu) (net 6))
 (segment (start 161.575 87.075) (end 161 86.5) (width 0.3) (layer F.Cu) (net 7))
 (segment (start 161.575 88.295) (end 161.575 87.075) (width 0.3) (layer F.Cu) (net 7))
 (segment (start 156.6 87.1) (end 156.6 87.9) (width 0.3) (layer F.Cu) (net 7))
 (segment (start 157.2 86.5) (end 156.6 87.1) (width 0.3) (layer F.Cu) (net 7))
 (segment (start 161 86.5) (end 157.2 86.5) (width 0.3) (layer F.Cu) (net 7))
 (segment (start 160.565 89.565) (end 160.25 89.25) (width 0.3) (layer F.Cu) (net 3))
 (segment (start 161.575 89.565) (end 160.565 89.565) (width 0.3) (layer F.Cu) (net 3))
 (segment (start 159.25 89.25) (end 159.2 89.2) (width 0.3) (layer F.Cu) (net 3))
 (segment (start 160.25 89.25) (end 159.25 89.25) (width 0.3) (layer F.Cu) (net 3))
 (segment (start 160.635 90.835) (end 160.6 90.8) (width 0.3) (layer F.Cu) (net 3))
 (segment (start 161.575 90.835) (end 160.635 90.835) (width 0.3) (layer F.Cu) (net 3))
 (segment (start 160.6 90.8) (end 160.585 90.835) (width 0.25) (layer F.Cu) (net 3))
 (segment (start 160.3 89.719998) (end 160.3 90.55) (width 0.3) (layer F.Cu) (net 3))
 (segment (start 160.25 89.669998) (end 160.3 89.719998) (width 0.3) (layer F.Cu) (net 3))
 (segment (start 160.25 89.25) (end 160.25 89.669998) (width 0.3) (layer F.Cu) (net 3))
 (segment (start 160.585 90.835) (end 161.575 90.835) (width 0.3) (layer F.Cu) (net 3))
 (segment (start 160.3 90.55) (end 160.585 90.835) (width 0.3) (layer F.Cu) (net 3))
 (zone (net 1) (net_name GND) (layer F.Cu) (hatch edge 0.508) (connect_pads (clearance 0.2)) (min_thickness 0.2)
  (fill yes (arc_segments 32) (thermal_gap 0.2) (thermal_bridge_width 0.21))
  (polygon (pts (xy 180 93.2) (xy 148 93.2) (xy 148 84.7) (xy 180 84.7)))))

